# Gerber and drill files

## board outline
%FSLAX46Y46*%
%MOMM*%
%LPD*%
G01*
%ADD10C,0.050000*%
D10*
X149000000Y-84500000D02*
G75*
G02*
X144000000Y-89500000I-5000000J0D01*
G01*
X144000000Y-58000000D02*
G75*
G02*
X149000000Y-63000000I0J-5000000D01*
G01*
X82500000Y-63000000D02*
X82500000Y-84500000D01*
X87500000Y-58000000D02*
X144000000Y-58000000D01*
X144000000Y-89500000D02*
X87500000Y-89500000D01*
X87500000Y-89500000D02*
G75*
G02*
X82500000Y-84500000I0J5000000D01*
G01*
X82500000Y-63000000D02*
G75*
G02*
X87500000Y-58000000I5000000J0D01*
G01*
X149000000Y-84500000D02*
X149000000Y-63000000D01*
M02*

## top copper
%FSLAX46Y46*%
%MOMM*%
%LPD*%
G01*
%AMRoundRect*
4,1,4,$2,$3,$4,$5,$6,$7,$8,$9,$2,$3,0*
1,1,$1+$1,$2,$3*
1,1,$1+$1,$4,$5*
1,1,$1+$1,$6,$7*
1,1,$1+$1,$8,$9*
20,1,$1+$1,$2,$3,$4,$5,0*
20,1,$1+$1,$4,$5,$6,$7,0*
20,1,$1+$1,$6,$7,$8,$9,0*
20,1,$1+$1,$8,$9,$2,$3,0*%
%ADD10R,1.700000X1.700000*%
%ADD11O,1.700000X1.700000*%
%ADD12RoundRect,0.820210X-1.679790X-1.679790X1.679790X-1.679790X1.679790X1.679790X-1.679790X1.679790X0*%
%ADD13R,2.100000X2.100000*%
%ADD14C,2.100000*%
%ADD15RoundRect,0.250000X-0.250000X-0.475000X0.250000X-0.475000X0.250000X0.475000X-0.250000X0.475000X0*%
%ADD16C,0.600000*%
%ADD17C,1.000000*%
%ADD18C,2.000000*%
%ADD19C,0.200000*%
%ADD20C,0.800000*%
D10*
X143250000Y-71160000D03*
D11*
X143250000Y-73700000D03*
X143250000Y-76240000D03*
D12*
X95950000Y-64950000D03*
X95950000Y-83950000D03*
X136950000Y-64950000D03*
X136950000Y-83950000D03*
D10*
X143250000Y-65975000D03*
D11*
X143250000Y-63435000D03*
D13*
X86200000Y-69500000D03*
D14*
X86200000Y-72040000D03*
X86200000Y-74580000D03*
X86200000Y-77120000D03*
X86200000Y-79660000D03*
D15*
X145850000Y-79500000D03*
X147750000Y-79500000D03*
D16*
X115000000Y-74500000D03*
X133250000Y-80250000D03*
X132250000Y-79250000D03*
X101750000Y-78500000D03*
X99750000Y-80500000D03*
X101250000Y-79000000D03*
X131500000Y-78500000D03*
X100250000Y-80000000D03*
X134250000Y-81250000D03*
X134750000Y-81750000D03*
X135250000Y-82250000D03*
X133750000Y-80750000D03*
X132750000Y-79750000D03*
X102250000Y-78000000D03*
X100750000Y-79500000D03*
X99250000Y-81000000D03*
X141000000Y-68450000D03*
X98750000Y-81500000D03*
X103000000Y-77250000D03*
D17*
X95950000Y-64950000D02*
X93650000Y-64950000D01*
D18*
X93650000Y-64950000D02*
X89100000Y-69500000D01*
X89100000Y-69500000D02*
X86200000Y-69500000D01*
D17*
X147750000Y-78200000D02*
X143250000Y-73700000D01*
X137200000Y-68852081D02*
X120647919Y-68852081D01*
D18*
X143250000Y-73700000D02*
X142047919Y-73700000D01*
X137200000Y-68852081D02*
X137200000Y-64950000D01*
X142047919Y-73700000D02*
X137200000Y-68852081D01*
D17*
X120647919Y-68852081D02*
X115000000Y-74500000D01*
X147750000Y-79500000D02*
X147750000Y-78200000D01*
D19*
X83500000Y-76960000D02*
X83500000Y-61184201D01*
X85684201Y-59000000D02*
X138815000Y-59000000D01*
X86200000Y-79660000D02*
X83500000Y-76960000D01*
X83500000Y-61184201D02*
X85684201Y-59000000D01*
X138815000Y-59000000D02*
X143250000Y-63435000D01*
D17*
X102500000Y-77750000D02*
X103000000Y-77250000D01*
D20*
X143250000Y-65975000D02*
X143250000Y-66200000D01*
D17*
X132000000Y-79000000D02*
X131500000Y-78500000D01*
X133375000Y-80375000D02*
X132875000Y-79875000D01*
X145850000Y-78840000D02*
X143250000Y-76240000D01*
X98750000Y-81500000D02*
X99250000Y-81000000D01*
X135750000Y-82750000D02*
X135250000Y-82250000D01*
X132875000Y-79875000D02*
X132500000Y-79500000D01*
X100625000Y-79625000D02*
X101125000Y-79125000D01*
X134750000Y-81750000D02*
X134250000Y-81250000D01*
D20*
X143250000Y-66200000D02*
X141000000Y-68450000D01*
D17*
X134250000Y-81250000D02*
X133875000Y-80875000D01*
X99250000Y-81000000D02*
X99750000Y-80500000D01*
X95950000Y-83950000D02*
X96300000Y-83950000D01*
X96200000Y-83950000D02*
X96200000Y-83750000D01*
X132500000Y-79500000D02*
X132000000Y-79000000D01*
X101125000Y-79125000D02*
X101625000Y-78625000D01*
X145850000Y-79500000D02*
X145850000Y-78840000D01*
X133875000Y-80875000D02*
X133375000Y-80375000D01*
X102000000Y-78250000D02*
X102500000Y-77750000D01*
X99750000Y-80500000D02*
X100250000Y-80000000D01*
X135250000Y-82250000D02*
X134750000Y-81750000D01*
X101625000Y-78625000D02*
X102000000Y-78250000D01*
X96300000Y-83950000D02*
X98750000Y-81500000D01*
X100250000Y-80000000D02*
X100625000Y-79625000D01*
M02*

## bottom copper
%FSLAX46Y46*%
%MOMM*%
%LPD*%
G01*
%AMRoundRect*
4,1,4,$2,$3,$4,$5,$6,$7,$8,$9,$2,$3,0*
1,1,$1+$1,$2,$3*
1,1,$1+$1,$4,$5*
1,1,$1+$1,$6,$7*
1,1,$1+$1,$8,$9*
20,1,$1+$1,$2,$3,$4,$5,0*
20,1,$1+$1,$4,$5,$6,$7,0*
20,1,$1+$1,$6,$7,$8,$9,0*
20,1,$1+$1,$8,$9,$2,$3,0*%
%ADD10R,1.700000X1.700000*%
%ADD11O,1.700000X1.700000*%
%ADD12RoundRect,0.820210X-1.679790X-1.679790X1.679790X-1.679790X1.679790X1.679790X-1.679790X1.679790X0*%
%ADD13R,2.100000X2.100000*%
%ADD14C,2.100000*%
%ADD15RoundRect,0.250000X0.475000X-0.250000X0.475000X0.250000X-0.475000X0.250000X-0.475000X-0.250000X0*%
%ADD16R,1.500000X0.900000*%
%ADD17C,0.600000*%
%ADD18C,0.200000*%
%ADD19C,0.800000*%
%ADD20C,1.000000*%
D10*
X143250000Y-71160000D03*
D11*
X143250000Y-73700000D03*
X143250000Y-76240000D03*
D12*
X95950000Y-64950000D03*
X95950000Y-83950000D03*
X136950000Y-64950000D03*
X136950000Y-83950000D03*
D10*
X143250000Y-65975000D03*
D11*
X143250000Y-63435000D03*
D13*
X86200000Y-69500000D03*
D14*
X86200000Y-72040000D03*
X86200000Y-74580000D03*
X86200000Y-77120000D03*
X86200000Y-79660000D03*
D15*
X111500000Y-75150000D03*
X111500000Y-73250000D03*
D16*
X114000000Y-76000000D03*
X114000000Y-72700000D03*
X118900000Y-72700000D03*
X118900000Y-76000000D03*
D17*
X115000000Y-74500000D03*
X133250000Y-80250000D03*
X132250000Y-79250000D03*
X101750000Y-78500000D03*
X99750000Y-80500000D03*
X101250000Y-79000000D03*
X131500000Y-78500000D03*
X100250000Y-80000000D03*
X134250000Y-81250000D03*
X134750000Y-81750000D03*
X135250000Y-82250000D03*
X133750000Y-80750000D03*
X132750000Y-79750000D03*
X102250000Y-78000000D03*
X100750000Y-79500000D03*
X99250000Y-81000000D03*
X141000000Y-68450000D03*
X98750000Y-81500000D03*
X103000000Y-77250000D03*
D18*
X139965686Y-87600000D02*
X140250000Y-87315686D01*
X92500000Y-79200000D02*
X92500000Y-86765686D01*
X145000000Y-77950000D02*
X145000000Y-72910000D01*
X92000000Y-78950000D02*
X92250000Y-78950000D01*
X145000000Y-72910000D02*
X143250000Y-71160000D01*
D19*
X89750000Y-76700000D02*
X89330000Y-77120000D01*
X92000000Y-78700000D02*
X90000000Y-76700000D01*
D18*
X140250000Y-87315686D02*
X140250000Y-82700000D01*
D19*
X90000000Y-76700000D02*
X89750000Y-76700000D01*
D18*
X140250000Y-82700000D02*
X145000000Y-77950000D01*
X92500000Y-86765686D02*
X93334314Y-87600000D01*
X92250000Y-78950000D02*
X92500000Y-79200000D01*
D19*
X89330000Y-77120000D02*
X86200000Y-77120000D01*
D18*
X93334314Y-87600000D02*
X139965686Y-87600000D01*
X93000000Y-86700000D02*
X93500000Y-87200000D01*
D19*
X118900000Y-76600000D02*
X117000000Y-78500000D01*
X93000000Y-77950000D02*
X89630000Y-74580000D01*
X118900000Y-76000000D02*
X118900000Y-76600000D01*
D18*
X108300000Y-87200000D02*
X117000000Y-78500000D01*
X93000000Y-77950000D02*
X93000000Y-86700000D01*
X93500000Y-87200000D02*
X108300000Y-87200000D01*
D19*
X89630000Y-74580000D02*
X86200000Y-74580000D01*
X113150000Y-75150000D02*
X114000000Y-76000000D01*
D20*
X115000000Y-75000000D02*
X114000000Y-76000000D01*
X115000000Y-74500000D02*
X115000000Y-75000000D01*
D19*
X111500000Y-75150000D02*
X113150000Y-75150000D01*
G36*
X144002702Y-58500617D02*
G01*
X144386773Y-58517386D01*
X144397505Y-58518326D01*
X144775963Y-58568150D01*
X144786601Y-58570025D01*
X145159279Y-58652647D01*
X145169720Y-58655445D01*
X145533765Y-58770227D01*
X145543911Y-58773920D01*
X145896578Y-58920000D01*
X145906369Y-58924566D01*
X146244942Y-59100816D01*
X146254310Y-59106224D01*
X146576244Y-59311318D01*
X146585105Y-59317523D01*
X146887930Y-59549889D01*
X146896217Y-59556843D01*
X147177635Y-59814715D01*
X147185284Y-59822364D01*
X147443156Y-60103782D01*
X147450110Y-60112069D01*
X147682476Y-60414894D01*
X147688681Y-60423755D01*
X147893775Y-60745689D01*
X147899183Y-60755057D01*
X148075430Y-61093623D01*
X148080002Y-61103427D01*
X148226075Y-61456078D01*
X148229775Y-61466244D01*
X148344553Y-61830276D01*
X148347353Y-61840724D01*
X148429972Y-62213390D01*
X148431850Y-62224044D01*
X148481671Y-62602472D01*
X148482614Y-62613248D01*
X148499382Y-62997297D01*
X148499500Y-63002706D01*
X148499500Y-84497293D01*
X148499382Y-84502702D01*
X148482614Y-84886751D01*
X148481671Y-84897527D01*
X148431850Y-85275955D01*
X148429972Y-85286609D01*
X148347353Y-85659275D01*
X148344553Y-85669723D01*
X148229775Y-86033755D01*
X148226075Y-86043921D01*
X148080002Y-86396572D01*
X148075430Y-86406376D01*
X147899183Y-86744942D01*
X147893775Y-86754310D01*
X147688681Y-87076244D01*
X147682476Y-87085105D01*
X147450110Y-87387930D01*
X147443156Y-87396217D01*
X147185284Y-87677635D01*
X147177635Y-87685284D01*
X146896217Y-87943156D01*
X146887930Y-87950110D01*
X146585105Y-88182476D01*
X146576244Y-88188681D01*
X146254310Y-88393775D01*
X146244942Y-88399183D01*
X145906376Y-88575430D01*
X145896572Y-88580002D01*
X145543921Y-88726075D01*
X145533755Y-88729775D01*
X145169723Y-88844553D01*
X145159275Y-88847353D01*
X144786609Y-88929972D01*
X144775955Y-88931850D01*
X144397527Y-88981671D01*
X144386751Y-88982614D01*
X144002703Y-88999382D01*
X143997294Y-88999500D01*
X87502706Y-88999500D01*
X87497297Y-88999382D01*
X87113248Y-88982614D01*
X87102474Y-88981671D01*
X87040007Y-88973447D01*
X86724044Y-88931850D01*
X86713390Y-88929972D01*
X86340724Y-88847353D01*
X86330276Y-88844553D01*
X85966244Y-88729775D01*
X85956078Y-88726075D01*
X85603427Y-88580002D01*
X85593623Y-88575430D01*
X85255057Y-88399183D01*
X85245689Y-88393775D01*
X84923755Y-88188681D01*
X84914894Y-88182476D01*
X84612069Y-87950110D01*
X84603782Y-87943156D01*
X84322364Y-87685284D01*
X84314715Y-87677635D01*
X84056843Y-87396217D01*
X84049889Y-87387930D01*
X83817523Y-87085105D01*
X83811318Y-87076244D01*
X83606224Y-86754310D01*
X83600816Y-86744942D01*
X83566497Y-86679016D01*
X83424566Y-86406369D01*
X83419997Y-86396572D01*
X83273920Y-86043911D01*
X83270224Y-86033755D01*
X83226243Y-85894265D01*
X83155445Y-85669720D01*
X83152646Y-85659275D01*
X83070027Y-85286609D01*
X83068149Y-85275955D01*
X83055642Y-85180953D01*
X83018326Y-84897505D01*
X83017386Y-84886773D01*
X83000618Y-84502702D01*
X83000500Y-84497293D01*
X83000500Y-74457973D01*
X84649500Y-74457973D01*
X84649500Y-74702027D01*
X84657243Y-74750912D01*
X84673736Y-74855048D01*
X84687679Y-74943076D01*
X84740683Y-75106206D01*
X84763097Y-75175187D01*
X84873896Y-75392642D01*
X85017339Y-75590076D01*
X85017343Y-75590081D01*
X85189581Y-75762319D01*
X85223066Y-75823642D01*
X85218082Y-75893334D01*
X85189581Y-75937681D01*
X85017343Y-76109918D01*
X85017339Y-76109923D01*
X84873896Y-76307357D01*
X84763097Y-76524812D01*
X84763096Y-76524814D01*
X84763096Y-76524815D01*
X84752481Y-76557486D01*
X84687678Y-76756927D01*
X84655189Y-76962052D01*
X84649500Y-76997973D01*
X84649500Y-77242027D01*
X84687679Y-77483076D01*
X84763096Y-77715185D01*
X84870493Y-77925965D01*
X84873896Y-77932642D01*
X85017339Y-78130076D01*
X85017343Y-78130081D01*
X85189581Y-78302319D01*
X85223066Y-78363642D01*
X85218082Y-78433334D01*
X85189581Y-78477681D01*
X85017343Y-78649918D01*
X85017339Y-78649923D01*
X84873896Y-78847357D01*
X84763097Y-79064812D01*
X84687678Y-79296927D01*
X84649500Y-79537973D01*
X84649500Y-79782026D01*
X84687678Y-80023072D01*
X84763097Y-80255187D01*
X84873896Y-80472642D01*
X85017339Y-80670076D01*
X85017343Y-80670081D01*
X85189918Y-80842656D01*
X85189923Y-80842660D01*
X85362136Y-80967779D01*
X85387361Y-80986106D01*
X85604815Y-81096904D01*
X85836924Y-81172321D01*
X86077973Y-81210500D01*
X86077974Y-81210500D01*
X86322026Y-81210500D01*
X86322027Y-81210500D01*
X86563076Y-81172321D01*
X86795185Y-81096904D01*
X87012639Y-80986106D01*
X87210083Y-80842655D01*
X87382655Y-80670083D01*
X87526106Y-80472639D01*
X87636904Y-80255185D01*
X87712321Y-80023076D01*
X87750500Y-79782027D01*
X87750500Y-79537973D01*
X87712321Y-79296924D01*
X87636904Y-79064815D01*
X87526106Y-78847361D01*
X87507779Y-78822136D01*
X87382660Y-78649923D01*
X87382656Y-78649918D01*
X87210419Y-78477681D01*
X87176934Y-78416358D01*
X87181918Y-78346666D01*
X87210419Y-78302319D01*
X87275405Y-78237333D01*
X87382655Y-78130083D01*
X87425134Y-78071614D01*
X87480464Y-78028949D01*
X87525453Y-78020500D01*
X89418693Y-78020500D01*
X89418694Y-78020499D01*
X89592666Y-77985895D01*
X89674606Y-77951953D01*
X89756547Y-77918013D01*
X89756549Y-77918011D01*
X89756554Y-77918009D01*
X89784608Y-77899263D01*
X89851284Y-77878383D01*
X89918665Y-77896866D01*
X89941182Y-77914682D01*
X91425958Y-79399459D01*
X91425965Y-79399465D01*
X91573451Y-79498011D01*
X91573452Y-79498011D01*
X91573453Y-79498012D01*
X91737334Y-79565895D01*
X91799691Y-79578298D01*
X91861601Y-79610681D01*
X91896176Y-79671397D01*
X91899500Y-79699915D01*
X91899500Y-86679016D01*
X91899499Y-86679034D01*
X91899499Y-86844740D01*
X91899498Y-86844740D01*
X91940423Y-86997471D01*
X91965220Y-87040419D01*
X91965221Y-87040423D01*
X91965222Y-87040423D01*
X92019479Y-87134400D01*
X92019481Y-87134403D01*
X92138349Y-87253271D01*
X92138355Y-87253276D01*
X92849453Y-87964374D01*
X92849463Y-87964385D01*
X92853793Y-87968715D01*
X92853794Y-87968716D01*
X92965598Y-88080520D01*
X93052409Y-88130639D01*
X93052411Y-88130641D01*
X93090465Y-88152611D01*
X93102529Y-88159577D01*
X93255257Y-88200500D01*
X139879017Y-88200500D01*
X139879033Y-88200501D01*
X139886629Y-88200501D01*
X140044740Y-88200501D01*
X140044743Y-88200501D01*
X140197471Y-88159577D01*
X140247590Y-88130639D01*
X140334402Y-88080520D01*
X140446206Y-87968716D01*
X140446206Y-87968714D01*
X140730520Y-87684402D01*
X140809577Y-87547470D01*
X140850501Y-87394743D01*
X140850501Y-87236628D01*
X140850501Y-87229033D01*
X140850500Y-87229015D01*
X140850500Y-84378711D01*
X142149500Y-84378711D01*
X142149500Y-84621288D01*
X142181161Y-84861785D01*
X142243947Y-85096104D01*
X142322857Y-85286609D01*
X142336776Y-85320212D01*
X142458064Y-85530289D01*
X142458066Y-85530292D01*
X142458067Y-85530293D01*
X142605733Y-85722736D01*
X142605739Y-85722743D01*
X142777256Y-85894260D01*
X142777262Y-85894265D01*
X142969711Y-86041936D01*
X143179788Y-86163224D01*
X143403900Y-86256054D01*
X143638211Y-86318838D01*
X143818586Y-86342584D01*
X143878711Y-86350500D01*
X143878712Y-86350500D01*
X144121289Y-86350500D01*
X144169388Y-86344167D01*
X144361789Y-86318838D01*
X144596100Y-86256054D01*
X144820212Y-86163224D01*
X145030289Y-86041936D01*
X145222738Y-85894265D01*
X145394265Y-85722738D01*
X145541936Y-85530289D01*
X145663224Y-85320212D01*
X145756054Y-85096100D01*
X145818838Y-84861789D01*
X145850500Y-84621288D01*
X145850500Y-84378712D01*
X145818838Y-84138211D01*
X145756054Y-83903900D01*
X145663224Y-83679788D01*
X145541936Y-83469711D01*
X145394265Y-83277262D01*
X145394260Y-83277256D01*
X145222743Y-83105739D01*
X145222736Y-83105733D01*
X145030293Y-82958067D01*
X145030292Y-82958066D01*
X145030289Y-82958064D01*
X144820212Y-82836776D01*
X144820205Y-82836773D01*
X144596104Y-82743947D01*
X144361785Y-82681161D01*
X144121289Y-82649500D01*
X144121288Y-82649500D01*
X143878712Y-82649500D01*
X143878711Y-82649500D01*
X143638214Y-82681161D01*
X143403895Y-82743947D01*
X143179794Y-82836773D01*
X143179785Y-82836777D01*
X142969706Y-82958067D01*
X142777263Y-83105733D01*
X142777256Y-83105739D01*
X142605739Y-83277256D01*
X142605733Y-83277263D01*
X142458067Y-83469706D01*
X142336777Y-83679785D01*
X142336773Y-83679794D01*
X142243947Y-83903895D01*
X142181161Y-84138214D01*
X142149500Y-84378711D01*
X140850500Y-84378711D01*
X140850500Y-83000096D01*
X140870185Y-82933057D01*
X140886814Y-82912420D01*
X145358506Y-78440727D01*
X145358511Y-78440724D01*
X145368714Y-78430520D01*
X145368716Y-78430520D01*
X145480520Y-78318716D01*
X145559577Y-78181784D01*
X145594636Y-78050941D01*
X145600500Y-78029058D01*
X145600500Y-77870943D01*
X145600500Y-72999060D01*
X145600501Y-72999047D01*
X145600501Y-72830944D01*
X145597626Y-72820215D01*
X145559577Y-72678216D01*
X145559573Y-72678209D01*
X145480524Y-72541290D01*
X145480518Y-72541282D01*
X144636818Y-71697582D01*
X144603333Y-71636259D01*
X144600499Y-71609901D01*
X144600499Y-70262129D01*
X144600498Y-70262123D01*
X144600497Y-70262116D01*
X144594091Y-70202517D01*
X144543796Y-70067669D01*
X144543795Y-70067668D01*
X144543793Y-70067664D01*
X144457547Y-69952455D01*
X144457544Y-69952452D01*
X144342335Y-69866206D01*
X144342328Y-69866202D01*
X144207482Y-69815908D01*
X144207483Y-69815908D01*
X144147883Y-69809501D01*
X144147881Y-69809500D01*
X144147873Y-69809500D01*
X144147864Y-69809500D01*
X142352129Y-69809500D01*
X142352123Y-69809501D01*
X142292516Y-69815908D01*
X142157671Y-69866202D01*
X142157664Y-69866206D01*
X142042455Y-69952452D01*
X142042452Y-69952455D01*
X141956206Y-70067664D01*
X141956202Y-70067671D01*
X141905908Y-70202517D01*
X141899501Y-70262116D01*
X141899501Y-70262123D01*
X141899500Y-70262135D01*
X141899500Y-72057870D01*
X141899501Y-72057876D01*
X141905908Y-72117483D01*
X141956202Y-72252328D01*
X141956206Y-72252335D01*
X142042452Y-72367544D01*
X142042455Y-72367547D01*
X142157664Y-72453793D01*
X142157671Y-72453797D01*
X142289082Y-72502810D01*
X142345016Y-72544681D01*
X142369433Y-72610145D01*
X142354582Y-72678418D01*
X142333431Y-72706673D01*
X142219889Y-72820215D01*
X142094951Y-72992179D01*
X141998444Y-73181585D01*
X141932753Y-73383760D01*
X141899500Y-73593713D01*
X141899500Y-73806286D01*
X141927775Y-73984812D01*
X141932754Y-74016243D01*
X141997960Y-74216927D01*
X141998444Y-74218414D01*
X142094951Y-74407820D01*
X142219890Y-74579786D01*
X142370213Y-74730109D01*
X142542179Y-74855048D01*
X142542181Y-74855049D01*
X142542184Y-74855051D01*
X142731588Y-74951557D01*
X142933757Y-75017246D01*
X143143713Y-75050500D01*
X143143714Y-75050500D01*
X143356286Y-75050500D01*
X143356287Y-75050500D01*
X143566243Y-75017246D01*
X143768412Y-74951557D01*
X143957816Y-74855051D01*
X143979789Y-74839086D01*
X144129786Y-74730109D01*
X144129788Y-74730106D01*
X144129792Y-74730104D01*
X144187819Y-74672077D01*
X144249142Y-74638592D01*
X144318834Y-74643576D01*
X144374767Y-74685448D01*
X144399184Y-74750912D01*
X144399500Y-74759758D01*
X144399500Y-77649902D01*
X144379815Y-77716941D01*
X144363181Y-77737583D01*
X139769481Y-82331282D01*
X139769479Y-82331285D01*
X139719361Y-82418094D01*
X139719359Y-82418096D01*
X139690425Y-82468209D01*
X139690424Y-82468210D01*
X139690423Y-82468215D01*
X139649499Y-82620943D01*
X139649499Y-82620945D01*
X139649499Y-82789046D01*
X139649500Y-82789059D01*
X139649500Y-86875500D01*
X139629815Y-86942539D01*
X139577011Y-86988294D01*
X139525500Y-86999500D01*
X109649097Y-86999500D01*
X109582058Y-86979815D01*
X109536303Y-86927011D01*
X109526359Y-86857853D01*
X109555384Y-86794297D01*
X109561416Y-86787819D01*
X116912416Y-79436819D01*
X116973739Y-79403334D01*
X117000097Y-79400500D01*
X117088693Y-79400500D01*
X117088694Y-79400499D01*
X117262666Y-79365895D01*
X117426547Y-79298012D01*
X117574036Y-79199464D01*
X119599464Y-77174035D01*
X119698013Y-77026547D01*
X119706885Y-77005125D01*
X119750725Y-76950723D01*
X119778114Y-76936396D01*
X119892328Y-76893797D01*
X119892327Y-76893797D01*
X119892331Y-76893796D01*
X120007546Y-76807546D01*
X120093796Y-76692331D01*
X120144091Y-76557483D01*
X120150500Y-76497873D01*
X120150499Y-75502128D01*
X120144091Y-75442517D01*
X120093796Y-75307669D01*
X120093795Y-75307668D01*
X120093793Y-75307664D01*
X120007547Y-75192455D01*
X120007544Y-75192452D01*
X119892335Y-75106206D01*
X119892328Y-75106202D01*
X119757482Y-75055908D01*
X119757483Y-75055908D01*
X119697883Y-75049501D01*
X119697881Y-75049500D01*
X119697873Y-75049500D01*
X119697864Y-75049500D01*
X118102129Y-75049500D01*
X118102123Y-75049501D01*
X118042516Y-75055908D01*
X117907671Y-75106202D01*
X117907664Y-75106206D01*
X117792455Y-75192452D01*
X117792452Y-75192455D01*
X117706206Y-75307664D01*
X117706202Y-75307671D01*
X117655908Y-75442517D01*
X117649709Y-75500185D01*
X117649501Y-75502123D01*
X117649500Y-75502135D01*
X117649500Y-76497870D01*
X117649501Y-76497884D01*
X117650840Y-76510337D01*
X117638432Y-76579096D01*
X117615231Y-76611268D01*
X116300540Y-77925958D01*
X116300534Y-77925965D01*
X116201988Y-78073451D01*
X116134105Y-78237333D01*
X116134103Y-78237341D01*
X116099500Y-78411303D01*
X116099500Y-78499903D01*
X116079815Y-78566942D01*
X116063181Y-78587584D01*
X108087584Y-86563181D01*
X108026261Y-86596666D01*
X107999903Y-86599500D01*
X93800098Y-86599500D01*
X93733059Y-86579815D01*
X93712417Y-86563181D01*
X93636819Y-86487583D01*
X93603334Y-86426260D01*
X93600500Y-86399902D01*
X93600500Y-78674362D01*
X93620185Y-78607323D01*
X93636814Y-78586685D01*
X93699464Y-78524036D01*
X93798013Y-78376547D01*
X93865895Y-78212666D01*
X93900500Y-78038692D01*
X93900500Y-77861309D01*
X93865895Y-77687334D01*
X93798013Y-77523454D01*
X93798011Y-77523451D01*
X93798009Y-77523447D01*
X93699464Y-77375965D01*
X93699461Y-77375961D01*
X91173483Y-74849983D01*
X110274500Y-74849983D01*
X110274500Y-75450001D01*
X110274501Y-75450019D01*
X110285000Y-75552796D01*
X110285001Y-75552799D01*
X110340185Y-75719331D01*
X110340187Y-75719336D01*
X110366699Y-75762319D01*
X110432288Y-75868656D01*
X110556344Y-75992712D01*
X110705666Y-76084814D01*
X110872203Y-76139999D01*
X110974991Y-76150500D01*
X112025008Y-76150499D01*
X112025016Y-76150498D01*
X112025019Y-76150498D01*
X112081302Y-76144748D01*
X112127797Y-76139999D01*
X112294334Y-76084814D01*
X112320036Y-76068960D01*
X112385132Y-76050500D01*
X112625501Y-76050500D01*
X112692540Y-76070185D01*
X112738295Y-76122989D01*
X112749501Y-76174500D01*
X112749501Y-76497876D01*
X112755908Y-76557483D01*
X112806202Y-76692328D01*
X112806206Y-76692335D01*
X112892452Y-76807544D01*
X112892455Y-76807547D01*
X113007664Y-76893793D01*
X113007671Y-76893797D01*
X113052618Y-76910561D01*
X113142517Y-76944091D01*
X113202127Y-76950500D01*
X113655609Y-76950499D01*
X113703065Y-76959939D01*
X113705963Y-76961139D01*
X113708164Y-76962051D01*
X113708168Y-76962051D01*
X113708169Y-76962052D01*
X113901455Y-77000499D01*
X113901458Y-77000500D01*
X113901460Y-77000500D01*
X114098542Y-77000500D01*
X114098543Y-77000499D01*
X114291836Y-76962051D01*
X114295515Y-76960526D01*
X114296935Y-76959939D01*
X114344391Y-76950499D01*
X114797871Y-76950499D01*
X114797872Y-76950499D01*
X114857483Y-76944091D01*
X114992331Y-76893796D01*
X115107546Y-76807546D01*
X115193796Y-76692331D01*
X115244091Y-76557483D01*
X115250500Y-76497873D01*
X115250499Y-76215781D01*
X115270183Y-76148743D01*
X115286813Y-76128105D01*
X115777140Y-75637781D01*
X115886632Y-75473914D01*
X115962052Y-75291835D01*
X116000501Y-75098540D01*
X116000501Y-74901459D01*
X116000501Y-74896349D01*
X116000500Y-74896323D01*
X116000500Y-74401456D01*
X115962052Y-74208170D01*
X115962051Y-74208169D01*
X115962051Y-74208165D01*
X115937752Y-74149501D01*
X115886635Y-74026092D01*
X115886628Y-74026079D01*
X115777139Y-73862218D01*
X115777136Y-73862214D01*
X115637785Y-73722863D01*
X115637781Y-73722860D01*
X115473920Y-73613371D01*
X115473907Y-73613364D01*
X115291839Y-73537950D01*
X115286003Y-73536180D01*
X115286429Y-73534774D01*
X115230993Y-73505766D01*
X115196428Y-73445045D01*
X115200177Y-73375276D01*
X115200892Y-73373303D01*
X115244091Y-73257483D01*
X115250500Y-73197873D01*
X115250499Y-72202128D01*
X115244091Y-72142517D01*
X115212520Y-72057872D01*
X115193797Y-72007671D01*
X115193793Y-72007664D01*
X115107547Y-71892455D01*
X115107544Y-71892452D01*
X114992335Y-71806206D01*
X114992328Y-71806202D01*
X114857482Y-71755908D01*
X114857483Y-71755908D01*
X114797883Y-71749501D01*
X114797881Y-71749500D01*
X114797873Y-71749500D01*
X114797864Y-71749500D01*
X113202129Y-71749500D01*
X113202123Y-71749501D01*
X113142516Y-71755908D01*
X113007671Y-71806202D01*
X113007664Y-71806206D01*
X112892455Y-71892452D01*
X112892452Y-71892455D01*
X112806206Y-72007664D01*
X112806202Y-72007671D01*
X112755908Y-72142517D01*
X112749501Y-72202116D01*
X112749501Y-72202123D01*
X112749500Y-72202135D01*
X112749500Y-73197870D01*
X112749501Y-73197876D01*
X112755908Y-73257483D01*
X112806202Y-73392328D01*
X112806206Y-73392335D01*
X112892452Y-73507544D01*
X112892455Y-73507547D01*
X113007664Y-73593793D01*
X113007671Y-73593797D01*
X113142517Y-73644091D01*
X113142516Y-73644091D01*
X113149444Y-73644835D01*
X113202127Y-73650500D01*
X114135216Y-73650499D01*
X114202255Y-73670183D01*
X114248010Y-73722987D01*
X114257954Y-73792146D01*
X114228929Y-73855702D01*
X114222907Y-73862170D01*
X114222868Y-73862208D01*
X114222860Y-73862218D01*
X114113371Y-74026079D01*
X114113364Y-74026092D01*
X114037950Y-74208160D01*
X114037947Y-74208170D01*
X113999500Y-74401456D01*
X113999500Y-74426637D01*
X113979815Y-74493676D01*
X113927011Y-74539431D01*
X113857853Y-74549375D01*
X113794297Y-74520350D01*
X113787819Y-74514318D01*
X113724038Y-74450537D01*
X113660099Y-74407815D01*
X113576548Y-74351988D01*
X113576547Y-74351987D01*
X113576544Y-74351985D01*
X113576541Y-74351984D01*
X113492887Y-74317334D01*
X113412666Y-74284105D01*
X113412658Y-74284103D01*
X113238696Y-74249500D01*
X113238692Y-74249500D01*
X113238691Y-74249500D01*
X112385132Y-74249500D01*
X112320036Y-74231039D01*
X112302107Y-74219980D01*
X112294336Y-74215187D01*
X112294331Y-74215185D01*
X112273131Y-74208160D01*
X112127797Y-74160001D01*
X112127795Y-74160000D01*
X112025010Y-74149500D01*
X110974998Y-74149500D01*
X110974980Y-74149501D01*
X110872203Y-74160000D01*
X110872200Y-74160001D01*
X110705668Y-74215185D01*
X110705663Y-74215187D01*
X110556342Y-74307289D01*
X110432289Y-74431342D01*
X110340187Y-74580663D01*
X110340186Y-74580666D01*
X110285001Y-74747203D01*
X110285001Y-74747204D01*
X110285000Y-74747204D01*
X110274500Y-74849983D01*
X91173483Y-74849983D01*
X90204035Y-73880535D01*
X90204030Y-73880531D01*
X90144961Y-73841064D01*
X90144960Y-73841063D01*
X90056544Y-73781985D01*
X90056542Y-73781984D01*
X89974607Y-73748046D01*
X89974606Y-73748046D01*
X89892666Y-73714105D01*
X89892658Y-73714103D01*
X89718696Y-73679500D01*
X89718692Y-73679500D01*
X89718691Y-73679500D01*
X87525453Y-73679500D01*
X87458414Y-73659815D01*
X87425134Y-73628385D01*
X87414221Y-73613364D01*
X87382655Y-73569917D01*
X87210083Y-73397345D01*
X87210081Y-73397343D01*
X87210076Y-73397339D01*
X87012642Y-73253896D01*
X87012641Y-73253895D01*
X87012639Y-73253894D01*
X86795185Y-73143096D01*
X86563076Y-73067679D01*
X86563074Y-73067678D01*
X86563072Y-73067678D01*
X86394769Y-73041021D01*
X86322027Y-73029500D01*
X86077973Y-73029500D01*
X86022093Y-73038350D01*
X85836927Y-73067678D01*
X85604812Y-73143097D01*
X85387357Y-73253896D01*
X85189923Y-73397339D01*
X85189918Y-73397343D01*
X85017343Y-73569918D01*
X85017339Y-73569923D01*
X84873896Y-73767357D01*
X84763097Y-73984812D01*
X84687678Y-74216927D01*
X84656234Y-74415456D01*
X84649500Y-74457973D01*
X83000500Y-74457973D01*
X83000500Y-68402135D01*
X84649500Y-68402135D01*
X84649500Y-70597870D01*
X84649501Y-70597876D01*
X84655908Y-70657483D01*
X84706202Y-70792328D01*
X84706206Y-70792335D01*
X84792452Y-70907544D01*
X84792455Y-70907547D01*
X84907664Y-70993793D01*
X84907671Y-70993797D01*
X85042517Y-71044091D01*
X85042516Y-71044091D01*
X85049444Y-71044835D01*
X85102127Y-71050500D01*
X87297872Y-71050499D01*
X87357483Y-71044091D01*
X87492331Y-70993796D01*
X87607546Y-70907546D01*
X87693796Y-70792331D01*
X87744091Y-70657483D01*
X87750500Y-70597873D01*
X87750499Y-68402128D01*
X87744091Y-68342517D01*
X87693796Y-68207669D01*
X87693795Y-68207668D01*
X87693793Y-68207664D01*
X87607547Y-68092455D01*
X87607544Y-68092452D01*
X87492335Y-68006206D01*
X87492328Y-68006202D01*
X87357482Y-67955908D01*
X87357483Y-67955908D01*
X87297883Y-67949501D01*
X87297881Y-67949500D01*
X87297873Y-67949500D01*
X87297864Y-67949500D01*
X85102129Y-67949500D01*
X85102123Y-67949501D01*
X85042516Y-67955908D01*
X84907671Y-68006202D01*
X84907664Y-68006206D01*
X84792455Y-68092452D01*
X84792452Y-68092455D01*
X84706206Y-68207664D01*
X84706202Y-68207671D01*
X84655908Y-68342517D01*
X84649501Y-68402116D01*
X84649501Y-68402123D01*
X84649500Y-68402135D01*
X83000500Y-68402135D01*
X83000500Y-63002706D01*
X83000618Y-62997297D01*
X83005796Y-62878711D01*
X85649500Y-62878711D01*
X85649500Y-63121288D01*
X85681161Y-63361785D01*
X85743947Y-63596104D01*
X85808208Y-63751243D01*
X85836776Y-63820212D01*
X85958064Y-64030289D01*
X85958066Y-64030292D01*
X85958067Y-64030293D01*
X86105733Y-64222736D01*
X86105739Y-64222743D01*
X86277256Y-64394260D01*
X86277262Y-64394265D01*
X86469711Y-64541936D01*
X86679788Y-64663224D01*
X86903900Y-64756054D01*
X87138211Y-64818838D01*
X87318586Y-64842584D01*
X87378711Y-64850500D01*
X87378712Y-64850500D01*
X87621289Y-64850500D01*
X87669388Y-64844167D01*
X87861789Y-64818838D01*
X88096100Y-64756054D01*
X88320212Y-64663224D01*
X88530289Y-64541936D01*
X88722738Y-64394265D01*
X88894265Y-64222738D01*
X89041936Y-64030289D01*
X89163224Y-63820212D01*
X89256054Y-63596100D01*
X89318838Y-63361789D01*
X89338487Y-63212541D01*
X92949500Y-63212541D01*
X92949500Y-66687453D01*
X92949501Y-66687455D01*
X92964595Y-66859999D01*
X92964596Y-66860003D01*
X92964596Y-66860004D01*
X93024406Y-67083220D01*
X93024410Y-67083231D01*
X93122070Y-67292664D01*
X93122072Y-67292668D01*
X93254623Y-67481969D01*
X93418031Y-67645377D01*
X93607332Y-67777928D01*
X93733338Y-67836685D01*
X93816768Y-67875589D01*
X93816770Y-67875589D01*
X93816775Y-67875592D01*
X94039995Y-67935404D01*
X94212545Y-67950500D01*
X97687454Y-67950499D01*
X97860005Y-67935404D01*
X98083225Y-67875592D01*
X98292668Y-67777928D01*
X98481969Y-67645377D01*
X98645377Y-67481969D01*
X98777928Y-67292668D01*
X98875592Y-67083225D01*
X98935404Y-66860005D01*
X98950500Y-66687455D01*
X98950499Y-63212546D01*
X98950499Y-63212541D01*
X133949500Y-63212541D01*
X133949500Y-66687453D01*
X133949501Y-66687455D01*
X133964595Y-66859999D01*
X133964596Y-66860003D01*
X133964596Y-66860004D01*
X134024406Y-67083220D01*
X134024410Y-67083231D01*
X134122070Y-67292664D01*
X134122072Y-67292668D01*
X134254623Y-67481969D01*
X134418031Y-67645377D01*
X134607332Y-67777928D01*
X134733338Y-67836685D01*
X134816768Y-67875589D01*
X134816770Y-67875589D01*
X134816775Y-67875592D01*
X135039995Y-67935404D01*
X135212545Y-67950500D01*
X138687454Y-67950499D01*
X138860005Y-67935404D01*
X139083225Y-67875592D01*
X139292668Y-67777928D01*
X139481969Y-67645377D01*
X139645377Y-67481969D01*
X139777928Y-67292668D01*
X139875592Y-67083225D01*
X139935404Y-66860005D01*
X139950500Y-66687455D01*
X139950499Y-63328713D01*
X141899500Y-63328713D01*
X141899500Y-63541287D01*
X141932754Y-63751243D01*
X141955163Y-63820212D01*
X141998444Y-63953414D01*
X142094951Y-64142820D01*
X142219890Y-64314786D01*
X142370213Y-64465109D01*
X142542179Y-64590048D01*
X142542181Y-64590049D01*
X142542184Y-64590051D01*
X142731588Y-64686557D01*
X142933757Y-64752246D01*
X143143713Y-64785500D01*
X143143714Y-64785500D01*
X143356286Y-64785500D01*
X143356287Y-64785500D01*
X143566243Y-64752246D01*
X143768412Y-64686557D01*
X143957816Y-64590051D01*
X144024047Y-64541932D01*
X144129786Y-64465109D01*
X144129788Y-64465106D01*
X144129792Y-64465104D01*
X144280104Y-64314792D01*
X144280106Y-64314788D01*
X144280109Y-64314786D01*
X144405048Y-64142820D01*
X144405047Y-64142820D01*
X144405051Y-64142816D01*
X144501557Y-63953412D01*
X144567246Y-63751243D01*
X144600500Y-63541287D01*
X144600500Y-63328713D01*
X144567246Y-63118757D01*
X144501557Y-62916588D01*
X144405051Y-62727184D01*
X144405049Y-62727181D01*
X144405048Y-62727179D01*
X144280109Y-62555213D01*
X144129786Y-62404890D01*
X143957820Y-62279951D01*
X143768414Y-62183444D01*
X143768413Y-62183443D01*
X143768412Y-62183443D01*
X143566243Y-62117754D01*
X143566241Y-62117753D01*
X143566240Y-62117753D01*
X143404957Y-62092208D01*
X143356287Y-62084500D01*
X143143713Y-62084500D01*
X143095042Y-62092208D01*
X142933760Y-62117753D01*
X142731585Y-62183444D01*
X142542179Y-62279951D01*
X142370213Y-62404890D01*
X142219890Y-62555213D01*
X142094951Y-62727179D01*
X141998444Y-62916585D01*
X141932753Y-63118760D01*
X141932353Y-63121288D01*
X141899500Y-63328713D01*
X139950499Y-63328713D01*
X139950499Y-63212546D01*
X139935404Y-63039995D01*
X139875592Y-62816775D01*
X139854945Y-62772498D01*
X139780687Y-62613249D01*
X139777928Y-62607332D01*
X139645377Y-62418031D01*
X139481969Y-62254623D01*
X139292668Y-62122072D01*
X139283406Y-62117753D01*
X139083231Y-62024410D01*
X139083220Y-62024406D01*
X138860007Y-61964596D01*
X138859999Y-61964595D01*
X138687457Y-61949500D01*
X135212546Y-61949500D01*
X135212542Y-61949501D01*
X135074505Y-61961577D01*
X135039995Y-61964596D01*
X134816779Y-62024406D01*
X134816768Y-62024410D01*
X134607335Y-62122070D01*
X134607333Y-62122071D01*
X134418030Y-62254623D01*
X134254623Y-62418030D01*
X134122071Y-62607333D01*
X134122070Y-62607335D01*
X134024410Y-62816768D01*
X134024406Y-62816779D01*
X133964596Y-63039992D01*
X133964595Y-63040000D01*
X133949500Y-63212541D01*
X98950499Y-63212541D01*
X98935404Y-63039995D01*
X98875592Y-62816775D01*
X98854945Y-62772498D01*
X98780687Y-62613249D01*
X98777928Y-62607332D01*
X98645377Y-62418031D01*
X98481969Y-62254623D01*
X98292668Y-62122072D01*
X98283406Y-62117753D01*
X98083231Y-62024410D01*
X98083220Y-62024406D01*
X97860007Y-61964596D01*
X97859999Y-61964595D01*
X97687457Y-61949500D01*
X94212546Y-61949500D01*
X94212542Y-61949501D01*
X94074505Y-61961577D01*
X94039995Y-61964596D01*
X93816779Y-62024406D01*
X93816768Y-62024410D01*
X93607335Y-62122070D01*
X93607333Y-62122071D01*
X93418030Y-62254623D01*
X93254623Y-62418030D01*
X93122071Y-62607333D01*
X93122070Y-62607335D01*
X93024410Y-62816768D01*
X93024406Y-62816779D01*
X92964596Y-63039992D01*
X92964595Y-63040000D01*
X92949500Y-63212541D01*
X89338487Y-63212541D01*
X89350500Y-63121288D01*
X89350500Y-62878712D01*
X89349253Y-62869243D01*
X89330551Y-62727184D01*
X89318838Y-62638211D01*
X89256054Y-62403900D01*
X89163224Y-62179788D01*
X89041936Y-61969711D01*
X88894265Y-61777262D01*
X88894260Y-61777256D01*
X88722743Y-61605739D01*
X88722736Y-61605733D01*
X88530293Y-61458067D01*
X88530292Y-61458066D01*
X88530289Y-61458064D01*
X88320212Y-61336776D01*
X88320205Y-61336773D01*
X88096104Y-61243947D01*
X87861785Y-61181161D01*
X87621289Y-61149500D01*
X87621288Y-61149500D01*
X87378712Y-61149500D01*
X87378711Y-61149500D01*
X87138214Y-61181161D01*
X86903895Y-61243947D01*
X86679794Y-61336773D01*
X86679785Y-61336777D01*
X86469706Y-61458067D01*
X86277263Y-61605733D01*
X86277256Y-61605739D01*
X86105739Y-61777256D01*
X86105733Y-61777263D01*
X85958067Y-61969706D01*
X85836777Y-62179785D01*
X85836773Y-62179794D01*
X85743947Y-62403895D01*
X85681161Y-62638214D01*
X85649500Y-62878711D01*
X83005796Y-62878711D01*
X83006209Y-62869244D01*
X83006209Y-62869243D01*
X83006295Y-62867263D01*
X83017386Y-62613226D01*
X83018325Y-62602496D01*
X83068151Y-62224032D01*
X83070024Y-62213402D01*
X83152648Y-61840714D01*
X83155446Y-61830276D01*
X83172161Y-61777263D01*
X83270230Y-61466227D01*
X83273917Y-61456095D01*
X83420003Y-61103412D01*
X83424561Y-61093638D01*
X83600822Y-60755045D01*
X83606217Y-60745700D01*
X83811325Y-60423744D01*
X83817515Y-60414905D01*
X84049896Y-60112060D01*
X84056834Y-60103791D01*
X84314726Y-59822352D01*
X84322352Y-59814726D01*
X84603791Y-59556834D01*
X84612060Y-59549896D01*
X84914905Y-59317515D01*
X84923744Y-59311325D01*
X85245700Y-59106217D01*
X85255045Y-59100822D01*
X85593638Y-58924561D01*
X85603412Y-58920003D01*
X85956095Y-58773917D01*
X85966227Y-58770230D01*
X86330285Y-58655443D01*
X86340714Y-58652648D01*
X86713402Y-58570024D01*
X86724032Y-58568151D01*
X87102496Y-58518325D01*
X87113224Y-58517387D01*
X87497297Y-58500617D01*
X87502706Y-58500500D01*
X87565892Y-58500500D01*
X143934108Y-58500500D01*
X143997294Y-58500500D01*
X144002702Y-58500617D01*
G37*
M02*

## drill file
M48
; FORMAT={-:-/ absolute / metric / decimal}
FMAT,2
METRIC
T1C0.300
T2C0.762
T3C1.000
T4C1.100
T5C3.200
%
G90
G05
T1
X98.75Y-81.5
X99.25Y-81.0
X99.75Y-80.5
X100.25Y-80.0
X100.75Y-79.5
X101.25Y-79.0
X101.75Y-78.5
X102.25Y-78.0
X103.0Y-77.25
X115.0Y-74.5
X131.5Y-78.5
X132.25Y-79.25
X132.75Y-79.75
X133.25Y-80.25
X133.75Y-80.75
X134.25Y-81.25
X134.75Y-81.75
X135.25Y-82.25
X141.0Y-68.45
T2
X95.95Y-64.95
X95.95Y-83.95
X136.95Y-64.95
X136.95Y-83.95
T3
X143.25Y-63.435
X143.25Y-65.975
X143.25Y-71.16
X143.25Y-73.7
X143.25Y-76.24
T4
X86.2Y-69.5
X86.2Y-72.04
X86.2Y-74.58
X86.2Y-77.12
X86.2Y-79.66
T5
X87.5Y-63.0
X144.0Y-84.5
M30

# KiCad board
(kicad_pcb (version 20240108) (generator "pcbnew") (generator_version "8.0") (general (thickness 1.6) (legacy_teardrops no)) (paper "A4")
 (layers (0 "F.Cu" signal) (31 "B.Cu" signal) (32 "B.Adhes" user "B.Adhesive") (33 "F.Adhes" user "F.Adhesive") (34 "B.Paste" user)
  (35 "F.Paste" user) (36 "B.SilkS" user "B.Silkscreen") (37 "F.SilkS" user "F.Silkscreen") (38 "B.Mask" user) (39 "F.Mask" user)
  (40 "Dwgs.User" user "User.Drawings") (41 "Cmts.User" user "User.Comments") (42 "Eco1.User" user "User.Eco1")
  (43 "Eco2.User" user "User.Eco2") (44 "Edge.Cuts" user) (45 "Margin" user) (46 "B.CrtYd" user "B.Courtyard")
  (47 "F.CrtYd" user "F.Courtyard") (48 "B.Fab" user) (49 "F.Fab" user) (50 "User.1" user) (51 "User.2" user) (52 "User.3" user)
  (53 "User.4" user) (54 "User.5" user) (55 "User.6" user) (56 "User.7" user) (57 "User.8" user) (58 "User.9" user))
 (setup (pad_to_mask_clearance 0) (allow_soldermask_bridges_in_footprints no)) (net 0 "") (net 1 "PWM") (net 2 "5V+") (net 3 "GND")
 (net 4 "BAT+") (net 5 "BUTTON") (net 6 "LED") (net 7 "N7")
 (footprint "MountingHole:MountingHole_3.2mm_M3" (layer "F.Cu") (at 87.5 63)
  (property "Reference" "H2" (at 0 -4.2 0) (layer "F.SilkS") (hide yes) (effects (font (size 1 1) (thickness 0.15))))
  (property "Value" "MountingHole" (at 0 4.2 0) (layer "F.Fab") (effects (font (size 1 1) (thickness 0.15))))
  (pad "" np_thru_hole circle (at 0 0) (size 3.2 3.2) (drill 3.2) (layers "*.Cu" "*.Mask")))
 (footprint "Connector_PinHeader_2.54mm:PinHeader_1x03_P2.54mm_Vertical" (layer "F.Cu") (at 143.25 71.16)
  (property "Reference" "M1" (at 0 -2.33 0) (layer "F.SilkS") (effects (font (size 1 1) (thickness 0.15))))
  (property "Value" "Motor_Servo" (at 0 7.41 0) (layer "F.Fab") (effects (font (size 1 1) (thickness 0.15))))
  (pad "1" thru_hole rect (at 0 0) (size 1.7 1.7) (drill 1) (layers "*.Cu" "*.Mask") (remove_unused_layers no) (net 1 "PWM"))
  (pad "2" thru_hole oval (at 0 2.54) (size 1.7 1.7) (drill 1) (layers "*.Cu" "*.Mask") (remove_unused_layers no) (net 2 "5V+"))
  (pad "3" thru_hole oval (at 0 5.08) (size 1.7 1.7) (drill 1) (layers "*.Cu" "*.Mask") (remove_unused_layers no) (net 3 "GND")))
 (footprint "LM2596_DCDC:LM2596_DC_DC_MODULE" (layer "F.Cu") (at 94.95 63.95)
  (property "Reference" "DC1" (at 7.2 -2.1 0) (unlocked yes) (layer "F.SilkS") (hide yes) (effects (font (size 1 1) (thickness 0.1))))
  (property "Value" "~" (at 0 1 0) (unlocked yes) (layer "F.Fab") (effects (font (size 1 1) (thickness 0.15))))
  (pad "0" thru_hole roundrect (at 1 1) (size 5 5) (drill oval 0.762) (layers "*.Cu" "*.Mask") (remove_unused_layers no)
   (roundrect_rratio 0.1640419948) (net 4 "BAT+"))
  (pad "1" thru_hole roundrect (at 1 20) (size 5 5) (drill oval 0.762) (layers "*.Cu" "*.Mask") (remove_unused_layers no)
   (roundrect_rratio 0.1640419948) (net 3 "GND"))
  (pad "2" thru_hole roundrect (at 42 1) (size 5 5) (drill oval 0.762) (layers "*.Cu" "*.Mask") (remove_unused_layers no)
   (roundrect_rratio 0.1640419948) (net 2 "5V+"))
  (pad "3" thru_hole roundrect (at 42 20) (size 5 5) (drill oval 0.762) (layers "*.Cu" "*.Mask") (remove_unused_layers no)
   (roundrect_rratio 0.1640419948) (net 3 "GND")))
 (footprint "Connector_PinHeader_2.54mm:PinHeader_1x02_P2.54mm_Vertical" (layer "F.Cu") (at 143.25 65.975 180)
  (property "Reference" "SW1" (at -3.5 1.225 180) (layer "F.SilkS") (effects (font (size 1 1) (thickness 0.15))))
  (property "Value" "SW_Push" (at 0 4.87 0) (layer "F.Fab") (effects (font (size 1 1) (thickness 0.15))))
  (pad "1" thru_hole rect (at 0 0 180) (size 1.7 1.7) (drill 1) (layers "*.Cu" "*.Mask") (remove_unused_layers no) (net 3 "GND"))
  (pad "2" thru_hole oval (at 0 2.54 180) (size 1.7 1.7) (drill 1) (layers "*.Cu" "*.Mask") (remove_unused_layers no) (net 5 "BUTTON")))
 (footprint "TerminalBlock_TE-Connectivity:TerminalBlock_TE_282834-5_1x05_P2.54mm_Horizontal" (layer "F.Cu") (at 86.2 69.5 -90)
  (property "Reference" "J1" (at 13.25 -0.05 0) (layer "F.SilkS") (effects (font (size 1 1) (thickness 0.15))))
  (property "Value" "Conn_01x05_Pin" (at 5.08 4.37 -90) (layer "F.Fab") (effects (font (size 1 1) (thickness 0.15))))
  (pad "1" thru_hole rect (at 0 0 270) (size 2.1 2.1) (drill 1.1) (layers "*.Cu" "*.Mask") (remove_unused_layers no) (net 4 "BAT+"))
  (pad "2" thru_hole circle (at 2.54 0 270) (size 2.1 2.1) (drill 1.1) (layers "*.Cu" "*.Mask") (remove_unused_layers no) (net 3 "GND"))
  (pad "3" thru_hole circle (at 5.08 0 270) (size 2.1 2.1) (drill 1.1) (layers "*.Cu" "*.Mask") (remove_unused_layers no) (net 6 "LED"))
  (pad "4" thru_hole circle (at 7.62 0 270) (size 2.1 2.1) (drill 1.1) (layers "*.Cu" "*.Mask") (remove_unused_layers no) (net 1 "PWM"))
  (pad "5" thru_hole circle (at 10.16 0 270) (size 2.1 2.1) (drill 1.1) (layers "*.Cu" "*.Mask") (remove_unused_layers no) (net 5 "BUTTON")))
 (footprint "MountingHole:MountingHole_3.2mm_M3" (layer "F.Cu") (at 144 84.5)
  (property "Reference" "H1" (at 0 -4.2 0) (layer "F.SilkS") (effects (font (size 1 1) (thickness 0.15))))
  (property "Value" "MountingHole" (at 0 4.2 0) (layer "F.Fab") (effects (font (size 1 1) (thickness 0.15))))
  (pad "" np_thru_hole circle (at 0 0) (size 3.2 3.2) (drill 3.2) (layers "*.Cu" "*.Mask")))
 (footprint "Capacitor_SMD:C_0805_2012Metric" (layer "F.Cu") (at 146.8 79.5)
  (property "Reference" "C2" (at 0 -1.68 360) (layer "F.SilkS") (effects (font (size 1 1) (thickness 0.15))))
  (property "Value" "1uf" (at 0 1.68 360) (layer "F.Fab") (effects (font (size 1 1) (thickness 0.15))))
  (pad "1" smd roundrect (at -0.95 0) (size 1 1.45) (layers "F.Cu" "F.Paste" "F.Mask") (roundrect_rratio 0.25) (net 3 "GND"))
  (pad "2" smd roundrect (at 0.95 0) (size 1 1.45) (layers "F.Cu" "F.Paste" "F.Mask") (roundrect_rratio 0.25) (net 2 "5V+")))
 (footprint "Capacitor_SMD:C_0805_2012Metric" (layer "B.Cu") (at 111.5 74.2 90)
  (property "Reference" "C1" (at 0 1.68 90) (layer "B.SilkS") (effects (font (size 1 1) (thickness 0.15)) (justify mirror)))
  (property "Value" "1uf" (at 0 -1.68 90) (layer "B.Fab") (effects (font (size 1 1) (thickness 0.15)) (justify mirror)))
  (pad "1" smd roundrect (at -0.95 0 90) (size 1 1.45) (layers "B.Cu" "B.Paste" "B.Mask") (roundrect_rratio 0.25) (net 2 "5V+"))
  (pad "2" smd roundrect (at 0.95 0 90) (size 1 1.45) (layers "B.Cu" "B.Paste" "B.Mask") (roundrect_rratio 0.25) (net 3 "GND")))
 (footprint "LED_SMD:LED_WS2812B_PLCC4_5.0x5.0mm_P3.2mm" (layer "B.Cu") (at 116.45 74.35)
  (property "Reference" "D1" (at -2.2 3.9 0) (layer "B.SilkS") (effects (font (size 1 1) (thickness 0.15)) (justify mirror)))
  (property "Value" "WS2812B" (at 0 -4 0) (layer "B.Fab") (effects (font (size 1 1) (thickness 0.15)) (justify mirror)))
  (pad "1" smd rect (at -2.45 1.65) (size 1.5 0.9) (layers "B.Cu" "B.Paste" "B.Mask") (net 2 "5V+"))
  (pad "2" smd rect (at -2.45 -1.65) (size 1.5 0.9) (layers "B.Cu" "B.Paste" "B.Mask") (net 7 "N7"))
  (pad "3" smd rect (at 2.45 -1.65) (size 1.5 0.9) (layers "B.Cu" "B.Paste" "B.Mask") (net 3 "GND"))
  (pad "4" smd rect (at 2.45 1.65) (size 1.5 0.9) (layers "B.Cu" "B.Paste" "B.Mask") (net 6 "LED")))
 (gr_arc (start 149 84.5) (mid 147.535534 88.035534) (end 144 89.5) (stroke (width 0.05) (type default)) (layer "Edge.Cuts"))
 (gr_arc (start 144 58) (mid 147.535534 59.464466) (end 149 63) (stroke (width 0.05) (type default)) (layer "Edge.Cuts"))
 (gr_line (start 82.5 63) (end 82.5 84.5) (stroke (width 0.05) (type default)) (layer "Edge.Cuts"))
 (gr_line (start 87.5 58) (end 144 58) (stroke (width 0.05) (type default)) (layer "Edge.Cuts"))
 (gr_line (start 144 89.5) (end 87.5 89.5) (stroke (width 0.05) (type default)) (layer "Edge.Cuts"))
 (gr_arc (start 87.5 89.5) (mid 83.964466 88.035534) (end 82.5 84.5) (stroke (width 0.05) (type default)) (layer "Edge.Cuts"))
 (gr_arc (start 82.5 63) (mid 83.964466 59.464466) (end 87.5 58) (stroke (width 0.05) (type default)) (layer "Edge.Cuts"))
 (gr_line (start 149 84.5) (end 149 63) (stroke (width 0.05) (type default)) (layer "Edge.Cuts"))
 (segment (start 95.95 64.95) (end 93.65 64.95) (width 1) (layer "F.Cu") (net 4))
 (segment (start 93.65 64.95) (end 89.1 69.5) (width 2) (layer "F.Cu") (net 4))
 (segment (start 89.1 69.5) (end 86.2 69.5) (width 2) (layer "F.Cu") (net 4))
 (segment (start 139.965686 87.6) (end 140.25 87.315686) (width 0.2) (layer "B.Cu") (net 1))
 (segment (start 92.5 79.2) (end 92.5 86.765686) (width 0.2) (layer "B.Cu") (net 1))
 (segment (start 145 77.95) (end 145 72.91) (width 0.2) (layer "B.Cu") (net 1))
 (segment (start 92 78.95) (end 92.25 78.95) (width 0.2) (layer "B.Cu") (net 1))
 (segment (start 145 72.91) (end 143.25 71.16) (width 0.2) (layer "B.Cu") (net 1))
 (segment (start 89.75 76.7) (end 89.33 77.12) (width 0.8) (layer "B.Cu") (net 1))
 (segment (start 92 78.7) (end 90 76.7) (width 0.8) (layer "B.Cu") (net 1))
 (segment (start 140.25 87.315686) (end 140.25 82.7) (width 0.2) (layer "B.Cu") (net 1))
 (segment (start 90 76.7) (end 89.75 76.7) (width 0.8) (layer "B.Cu") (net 1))
 (segment (start 140.25 82.7) (end 145 77.95) (width 0.2) (layer "B.Cu") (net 1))
 (segment (start 92.5 86.765686) (end 93.334314 87.6) (width 0.2) (layer "B.Cu") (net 1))
 (segment (start 92.25 78.95) (end 92.5 79.2) (width 0.2) (layer "B.Cu") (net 1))
 (segment (start 89.33 77.12) (end 86.2 77.12) (width 0.8) (layer "B.Cu") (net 1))
 (segment (start 93.334314 87.6) (end 139.965686 87.6) (width 0.2) (layer "B.Cu") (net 1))
 (segment (start 93 86.7) (end 93.5 87.2) (width 0.2) (layer "B.Cu") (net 6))
 (segment (start 118.9 76.6) (end 117 78.5) (width 0.8) (layer "B.Cu") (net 6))
 (segment (start 93 77.95) (end 89.63 74.58) (width 0.8) (layer "B.Cu") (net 6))
 (segment (start 118.9 76) (end 118.9 76.6) (width 0.8) (layer "B.Cu") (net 6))
 (segment (start 108.3 87.2) (end 117 78.5) (width 0.2) (layer "B.Cu") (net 6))
 (segment (start 93 77.95) (end 93 86.7) (width 0.2) (layer "B.Cu") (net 6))
 (segment (start 93.5 87.2) (end 108.3 87.2) (width 0.2) (layer "B.Cu") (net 6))
 (segment (start 89.63 74.58) (end 86.2 74.58) (width 0.8) (layer "B.Cu") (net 6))
 (segment (start 147.75 78.2) (end 143.25 73.7) (width 1) (layer "F.Cu") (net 2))
 (segment (start 137.2 68.852081) (end 120.647919 68.852081) (width 1) (layer "F.Cu") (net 2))
 (segment (start 143.25 73.7) (end 142.047919 73.7) (width 2) (layer "F.Cu") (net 2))
 (segment (start 137.2 68.852081) (end 137.2 64.95) (width 2) (layer "F.Cu") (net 2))
 (segment (start 142.047919 73.7) (end 137.2 68.852081) (width 2) (layer "F.Cu") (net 2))
 (segment (start 120.647919 68.852081) (end 115 74.5) (width 1) (layer "F.Cu") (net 2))
 (segment (start 147.75 79.5) (end 147.75 78.2) (width 1) (layer "F.Cu") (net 2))
 (via (at 115 74.5) (size 0.6) (drill 0.3) (layers "F.Cu" "B.Cu") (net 2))
 (segment (start 113.15 75.15) (end 114 76) (width 0.8) (layer "B.Cu") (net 2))
 (segment (start 115 75) (end 114 76) (width 1) (layer "B.Cu") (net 2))
 (segment (start 115 74.5) (end 115 75) (width 1) (layer "B.Cu") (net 2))
 (segment (start 111.5 75.15) (end 113.15 75.15) (width 0.8) (layer "B.Cu") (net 2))
 (segment (start 83.5 76.96) (end 83.5 61.184201) (width 0.2) (layer "F.Cu") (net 5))
 (segment (start 85.684201 59) (end 138.815 59) (width 0.2) (layer "F.Cu") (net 5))
 (segment (start 86.2 79.66) (end 83.5 76.96) (width 0.2) (layer "F.Cu") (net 5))
 (segment (start 83.5 61.184201) (end 85.684201 59) (width 0.2) (layer "F.Cu") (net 5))
 (segment (start 138.815 59) (end 143.25 63.435) (width 0.2) (layer "F.Cu") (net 5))
 (segment (start 102.5 77.75) (end 103 77.25) (width 1) (layer "F.Cu") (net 3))
 (segment (start 143.25 65.975) (end 143.25 66.2) (width 0.8) (layer "F.Cu") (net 3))
 (segment (start 132 79) (end 131.5 78.5) (width 1) (layer "F.Cu") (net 3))
 (segment (start 133.375 80.375) (end 132.875 79.875) (width 1) (layer "F.Cu") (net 3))
 (segment (start 145.85 78.84) (end 143.25 76.24) (width 1) (layer "F.Cu") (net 3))
 (segment (start 98.75 81.5) (end 99.25 81) (width 1) (layer "F.Cu") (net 3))
 (segment (start 135.75 82.75) (end 135.25 82.25) (width 1) (layer "F.Cu") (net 3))
 (segment (start 132.875 79.875) (end 132.5 79.5) (width 1) (layer "F.Cu") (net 3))
 (segment (start 100.625 79.625) (end 101.125 79.125) (width 1) (layer "F.Cu") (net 3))
 (segment (start 134.75 81.75) (end 134.25 81.25) (width 1) (layer "F.Cu") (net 3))
 (segment (start 143.25 66.2) (end 141 68.45) (width 0.8) (layer "F.Cu") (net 3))
 (segment (start 134.25 81.25) (end 133.875 80.875) (width 1) (layer "F.Cu") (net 3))
 (segment (start 99.25 81) (end 99.75 80.5) (width 1) (layer "F.Cu") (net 3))
 (segment (start 95.95 83.95) (end 96.3 83.95) (width 1) (layer "F.Cu") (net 3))
 (segment (start 96.2 83.95) (end 96.2 83.75) (width 1) (layer "F.Cu") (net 3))
 (segment (start 132.5 79.5) (end 132 79) (width 1) (layer "F.Cu") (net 3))
 (segment (start 101.125 79.125) (end 101.625 78.625) (width 1) (layer "F.Cu") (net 3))
 (segment (start 145.85 79.5) (end 145.85 78.84) (width 1) (layer "F.Cu") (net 3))
 (segment (start 133.875 80.875) (end 133.375 80.375) (width 1) (layer "F.Cu") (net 3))
 (segment (start 102 78.25) (end 102.5 77.75) (width 1) (layer "F.Cu") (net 3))
 (segment (start 99.75 80.5) (end 100.25 80) (width 1) (layer "F.Cu") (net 3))
 (segment (start 135.25 82.25) (end 134.75 81.75) (width 1) (layer "F.Cu") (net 3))
 (segment (start 101.625 78.625) (end 102 78.25) (width 1) (layer "F.Cu") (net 3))
 (segment (start 96.3 83.95) (end 98.75 81.5) (width 1) (layer "F.Cu") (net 3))
 (segment (start 100.25 80) (end 100.625 79.625) (width 1) (layer "F.Cu") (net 3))
 (via (at 133.25 80.25) (size 0.6) (drill 0.3) (layers "F.Cu" "B.Cu") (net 3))
 (via (at 132.25 79.25) (size 0.6) (drill 0.3) (layers "F.Cu" "B.Cu") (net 3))
 (via (at 101.75 78.5) (size 0.6) (drill 0.3) (layers "F.Cu" "B.Cu") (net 3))
 (via (at 99.75 80.5) (size 0.6) (drill 0.3) (layers "F.Cu" "B.Cu") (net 3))
 (via (at 101.25 79) (size 0.6) (drill 0.3) (layers "F.Cu" "B.Cu") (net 3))
 (via (at 131.5 78.5) (size 0.6) (drill 0.3) (layers "F.Cu" "B.Cu") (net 3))
 (via (at 100.25 80) (size 0.6) (drill 0.3) (layers "F.Cu" "B.Cu") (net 3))
 (via (at 134.25 81.25) (size 0.6) (drill 0.3) (layers "F.Cu" "B.Cu") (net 3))
 (via (at 134.75 81.75) (size 0.6) (drill 0.3) (layers "F.Cu" "B.Cu") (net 3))
 (via (at 135.25 82.25) (size 0.6) (drill 0.3) (layers "F.Cu" "B.Cu") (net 3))
 (via (at 133.75 80.75) (size 0.6) (drill 0.3) (layers "F.Cu" "B.Cu") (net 3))
 (via (at 132.75 79.75) (size 0.6) (drill 0.3) (layers "F.Cu" "B.Cu") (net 3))
 (via (at 102.25 78) (size 0.6) (drill 0.3) (layers "F.Cu" "B.Cu") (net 3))
 (via (at 100.75 79.5) (size 0.6) (drill 0.3) (layers "F.Cu" "B.Cu") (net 3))
 (via (at 99.25 81) (size 0.6) (drill 0.3) (layers "F.Cu" "B.Cu") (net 3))
 (via (at 141 68.45) (size 0.6) (drill 0.3) (layers "F.Cu" "B.Cu") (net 3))
 (via (at 98.75 81.5) (size 0.6) (drill 0.3) (layers "F.Cu" "B.Cu") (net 3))
 (via (at 103 77.25) (size 0.6) (drill 0.3) (layers "F.Cu" "B.Cu") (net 3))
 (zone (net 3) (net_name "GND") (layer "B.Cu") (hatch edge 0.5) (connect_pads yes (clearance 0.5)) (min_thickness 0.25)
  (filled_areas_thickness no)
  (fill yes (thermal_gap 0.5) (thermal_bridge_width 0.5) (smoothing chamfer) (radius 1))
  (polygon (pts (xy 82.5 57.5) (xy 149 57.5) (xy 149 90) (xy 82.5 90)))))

